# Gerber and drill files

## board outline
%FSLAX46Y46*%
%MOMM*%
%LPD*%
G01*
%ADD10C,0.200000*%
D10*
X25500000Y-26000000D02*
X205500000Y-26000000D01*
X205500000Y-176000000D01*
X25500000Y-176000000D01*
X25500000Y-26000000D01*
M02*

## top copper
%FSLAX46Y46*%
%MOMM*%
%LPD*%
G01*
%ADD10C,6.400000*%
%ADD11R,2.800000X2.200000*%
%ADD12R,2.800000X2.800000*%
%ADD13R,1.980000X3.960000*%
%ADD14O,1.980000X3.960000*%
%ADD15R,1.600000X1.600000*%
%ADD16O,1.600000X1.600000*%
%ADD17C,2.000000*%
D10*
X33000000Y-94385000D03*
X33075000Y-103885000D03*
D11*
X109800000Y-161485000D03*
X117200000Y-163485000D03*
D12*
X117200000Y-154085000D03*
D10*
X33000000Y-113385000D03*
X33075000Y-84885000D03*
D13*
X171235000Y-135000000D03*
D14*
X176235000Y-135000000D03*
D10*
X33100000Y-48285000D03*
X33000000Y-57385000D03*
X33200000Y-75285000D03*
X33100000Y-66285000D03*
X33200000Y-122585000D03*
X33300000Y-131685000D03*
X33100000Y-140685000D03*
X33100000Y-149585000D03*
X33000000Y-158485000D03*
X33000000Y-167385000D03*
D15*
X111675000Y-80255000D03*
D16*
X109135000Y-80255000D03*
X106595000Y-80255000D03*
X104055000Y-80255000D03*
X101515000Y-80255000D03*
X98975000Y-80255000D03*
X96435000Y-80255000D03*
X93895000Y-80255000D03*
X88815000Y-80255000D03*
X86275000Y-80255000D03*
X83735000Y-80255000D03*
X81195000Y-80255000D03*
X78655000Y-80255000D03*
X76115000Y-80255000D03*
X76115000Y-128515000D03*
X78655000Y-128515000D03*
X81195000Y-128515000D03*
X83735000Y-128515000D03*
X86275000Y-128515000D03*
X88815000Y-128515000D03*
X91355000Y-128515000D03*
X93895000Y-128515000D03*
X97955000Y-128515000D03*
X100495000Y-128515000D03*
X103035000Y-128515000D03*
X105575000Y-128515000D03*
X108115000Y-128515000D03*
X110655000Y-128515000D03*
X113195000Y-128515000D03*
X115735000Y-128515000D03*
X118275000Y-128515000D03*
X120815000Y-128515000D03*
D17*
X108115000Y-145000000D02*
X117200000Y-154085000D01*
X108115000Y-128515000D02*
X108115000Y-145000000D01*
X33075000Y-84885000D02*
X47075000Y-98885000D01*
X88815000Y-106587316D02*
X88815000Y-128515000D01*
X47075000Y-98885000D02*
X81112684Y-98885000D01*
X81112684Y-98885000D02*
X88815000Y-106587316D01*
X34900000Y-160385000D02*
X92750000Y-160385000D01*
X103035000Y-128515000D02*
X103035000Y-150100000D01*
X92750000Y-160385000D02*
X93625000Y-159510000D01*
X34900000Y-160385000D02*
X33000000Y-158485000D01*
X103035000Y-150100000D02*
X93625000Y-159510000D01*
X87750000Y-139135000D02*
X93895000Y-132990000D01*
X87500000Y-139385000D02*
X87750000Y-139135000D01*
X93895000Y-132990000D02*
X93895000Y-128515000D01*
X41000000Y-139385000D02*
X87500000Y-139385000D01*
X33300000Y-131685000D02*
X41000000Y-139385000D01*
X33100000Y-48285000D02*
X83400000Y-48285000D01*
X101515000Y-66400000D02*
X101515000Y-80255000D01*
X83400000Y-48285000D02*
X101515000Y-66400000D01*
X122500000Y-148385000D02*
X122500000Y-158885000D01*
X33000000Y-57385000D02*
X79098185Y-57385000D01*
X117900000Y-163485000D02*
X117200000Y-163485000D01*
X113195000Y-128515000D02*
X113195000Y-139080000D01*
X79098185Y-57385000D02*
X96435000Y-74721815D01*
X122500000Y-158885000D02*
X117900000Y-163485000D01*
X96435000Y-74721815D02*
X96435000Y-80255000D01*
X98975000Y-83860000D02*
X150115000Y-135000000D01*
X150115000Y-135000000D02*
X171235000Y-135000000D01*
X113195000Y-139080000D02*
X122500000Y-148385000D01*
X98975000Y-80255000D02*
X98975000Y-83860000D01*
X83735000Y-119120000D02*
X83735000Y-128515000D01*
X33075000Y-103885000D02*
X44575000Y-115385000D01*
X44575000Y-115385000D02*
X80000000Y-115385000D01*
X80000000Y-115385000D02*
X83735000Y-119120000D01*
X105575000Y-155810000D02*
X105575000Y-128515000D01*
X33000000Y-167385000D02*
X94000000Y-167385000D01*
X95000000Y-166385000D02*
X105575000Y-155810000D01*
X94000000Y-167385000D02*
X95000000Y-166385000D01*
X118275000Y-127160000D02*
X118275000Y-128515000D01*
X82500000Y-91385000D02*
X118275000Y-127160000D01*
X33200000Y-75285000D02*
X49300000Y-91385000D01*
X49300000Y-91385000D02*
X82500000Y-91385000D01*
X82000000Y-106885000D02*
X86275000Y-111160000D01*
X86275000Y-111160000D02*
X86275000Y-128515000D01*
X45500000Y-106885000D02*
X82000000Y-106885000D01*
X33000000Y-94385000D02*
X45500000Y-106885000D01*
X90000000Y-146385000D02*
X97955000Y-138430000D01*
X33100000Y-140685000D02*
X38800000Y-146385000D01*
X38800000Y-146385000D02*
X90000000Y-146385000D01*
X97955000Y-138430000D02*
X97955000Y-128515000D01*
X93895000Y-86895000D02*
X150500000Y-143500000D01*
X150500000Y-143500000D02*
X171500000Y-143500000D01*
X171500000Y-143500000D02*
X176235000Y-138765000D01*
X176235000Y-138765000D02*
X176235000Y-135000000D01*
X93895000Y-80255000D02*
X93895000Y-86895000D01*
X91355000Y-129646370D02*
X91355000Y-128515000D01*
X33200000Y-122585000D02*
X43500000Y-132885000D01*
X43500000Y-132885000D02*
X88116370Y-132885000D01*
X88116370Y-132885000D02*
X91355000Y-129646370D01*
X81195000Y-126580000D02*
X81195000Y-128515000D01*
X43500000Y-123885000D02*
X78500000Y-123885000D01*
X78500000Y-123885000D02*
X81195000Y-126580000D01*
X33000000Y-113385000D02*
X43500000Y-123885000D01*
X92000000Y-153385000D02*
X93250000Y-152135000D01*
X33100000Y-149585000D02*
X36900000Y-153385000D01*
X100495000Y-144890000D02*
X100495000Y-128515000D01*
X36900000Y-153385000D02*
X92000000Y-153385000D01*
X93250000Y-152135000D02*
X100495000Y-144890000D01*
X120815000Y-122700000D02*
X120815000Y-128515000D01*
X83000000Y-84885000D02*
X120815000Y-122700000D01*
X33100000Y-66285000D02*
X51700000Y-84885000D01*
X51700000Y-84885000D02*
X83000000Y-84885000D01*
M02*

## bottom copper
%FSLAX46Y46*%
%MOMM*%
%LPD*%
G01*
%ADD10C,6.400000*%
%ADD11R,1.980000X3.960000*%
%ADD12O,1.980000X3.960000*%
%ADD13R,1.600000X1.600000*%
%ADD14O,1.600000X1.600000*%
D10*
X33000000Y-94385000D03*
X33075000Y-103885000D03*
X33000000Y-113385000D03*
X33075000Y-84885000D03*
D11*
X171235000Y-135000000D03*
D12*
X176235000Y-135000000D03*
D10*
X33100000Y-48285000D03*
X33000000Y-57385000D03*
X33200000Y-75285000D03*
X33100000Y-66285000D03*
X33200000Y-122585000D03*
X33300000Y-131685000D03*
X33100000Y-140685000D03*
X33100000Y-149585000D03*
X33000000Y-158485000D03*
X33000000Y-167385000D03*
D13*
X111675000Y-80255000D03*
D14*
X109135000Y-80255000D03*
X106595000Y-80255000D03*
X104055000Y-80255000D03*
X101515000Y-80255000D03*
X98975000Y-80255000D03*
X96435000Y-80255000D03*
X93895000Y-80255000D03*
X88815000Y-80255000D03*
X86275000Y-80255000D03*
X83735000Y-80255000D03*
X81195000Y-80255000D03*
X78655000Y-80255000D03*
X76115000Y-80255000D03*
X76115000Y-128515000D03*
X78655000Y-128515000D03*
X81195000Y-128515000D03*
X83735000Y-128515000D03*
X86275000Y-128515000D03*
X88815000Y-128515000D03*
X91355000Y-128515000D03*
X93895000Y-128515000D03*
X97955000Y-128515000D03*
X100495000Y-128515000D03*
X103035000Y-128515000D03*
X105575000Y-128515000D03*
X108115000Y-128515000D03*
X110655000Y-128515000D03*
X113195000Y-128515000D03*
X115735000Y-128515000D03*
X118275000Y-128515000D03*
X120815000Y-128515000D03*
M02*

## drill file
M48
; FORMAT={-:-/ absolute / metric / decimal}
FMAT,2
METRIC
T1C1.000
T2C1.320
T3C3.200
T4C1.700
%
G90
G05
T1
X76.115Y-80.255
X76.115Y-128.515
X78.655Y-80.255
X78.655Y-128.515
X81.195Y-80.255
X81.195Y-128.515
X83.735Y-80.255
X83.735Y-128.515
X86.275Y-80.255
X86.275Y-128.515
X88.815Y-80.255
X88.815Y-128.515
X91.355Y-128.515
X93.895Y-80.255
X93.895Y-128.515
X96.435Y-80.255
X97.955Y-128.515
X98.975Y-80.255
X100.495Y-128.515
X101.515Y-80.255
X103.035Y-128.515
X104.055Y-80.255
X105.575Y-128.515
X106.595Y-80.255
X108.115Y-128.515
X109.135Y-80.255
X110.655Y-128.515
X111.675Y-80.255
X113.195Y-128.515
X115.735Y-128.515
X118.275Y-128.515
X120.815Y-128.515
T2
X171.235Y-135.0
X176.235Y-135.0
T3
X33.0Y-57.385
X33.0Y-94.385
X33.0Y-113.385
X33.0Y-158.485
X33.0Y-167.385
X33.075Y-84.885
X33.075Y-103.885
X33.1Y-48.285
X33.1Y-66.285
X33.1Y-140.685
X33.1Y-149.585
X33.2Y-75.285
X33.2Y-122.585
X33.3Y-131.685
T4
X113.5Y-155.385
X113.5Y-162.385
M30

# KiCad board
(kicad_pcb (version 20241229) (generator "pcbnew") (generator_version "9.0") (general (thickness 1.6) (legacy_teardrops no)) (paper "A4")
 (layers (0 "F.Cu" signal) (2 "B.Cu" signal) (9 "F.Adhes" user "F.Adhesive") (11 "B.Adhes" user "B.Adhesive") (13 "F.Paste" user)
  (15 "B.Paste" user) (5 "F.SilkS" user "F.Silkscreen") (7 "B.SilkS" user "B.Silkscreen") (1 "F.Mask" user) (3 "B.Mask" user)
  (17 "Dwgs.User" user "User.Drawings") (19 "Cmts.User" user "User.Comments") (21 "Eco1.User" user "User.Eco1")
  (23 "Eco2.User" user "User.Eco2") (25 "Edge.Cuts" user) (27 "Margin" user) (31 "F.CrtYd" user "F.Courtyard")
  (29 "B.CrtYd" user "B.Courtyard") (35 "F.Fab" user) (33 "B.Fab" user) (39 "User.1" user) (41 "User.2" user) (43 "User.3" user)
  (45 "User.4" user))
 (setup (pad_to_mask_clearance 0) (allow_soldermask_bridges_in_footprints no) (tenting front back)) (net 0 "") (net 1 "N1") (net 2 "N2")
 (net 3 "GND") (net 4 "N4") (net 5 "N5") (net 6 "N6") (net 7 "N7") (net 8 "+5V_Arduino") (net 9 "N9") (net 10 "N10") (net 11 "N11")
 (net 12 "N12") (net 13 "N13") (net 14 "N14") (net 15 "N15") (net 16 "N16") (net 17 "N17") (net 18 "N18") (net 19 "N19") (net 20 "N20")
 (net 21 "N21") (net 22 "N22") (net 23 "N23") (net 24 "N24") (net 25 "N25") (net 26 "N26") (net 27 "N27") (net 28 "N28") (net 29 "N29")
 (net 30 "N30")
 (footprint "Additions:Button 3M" (layer "F.Cu") (at 36.8 94.485)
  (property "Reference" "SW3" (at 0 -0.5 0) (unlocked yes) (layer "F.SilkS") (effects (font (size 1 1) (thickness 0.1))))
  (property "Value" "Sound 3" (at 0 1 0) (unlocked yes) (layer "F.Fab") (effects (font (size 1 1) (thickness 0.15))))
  (pad "2" thru_hole circle (at -3.8 -0.1) (size 6.4 6.4) (drill 3.2) (layers "*.Cu" "*.Mask") (remove_unused_layers no) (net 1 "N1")
   (zone_connect 2)))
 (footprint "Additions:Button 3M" (layer "F.Cu") (at 36.875 103.985)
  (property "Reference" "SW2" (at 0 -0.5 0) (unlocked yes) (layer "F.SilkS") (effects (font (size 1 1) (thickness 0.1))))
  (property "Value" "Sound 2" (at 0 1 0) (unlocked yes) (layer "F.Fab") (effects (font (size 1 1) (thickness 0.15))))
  (pad "2" thru_hole circle (at -3.8 -0.1) (size 6.4 6.4) (drill 3.2) (layers "*.Cu" "*.Mask") (remove_unused_layers no) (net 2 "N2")
   (zone_connect 2)))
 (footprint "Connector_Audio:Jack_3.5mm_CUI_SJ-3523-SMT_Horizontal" (layer "F.Cu") (at 113.5 159.885 180)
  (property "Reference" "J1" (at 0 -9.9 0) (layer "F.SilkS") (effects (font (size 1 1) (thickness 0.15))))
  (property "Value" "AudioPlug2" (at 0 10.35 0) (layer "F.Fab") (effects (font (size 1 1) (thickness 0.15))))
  (pad "" np_thru_hole circle (at 0 -2.5 180) (size 1.7 1.7) (drill 1.7) (layers "*.Cu" "*.Mask"))
  (pad "" np_thru_hole circle (at 0 4.5 180) (size 1.7 1.7) (drill 1.7) (layers "*.Cu" "*.Mask"))
  (pad "R" smd rect (at 3.7 -1.6 180) (size 2.8 2.2) (layers "F.Cu" "F.Mask" "F.Paste"))
  (pad "S" smd rect (at -3.7 -3.6 180) (size 2.8 2.2) (layers "F.Cu" "F.Mask" "F.Paste") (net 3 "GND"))
  (pad "T" smd rect (at -3.7 5.8 180) (size 2.8 2.8) (layers "F.Cu" "F.Mask" "F.Paste") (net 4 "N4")))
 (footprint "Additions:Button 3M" (layer "F.Cu") (at 36.8 113.485)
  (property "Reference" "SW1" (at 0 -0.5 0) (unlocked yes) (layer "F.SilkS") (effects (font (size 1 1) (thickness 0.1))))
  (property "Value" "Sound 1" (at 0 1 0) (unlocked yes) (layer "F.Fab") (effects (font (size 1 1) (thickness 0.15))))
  (pad "2" thru_hole circle (at -3.8 -0.1) (size 6.4 6.4) (drill 3.2) (layers "*.Cu" "*.Mask") (remove_unused_layers no) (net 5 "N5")
   (zone_connect 2)))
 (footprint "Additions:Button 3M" (layer "F.Cu") (at 36.875 84.985)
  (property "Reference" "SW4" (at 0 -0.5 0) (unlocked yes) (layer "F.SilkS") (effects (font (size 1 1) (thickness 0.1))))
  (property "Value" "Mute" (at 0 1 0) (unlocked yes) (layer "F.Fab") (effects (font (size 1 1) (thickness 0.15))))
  (pad "2" thru_hole circle (at -3.8 -0.1) (size 6.4 6.4) (drill 3.2) (layers "*.Cu" "*.Mask") (remove_unused_layers no) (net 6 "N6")
   (zone_connect 2)))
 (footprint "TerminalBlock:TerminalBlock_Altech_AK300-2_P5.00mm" (layer "F.Cu") (at 171.235 135)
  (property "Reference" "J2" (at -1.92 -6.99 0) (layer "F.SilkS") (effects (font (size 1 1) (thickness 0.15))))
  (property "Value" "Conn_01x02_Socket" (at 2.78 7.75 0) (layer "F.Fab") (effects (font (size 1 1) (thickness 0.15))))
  (pad "1" thru_hole rect (at 0 0) (size 1.98 3.96) (drill 1.32) (layers "*.Cu" "*.Mask") (remove_unused_layers no) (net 3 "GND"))
  (pad "2" thru_hole oval (at 5 0) (size 1.98 3.96) (drill 1.32) (layers "*.Cu" "*.Mask") (remove_unused_layers no) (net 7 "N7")))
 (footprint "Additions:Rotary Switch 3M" (layer "F.Cu") (at 33 63.785 90)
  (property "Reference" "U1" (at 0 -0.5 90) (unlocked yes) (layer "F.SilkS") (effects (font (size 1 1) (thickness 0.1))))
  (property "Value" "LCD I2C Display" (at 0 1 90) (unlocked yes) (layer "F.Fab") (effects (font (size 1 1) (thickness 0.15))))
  (pad "1" thru_hole circle (at 15.5 0.1 90) (size 6.4 6.4) (drill 3.2) (layers "*.Cu" "*.Mask") (remove_unused_layers no)
   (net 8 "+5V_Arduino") (zone_connect 2))
  (pad "2" thru_hole circle (at 6.4 0 90) (size 6.4 6.4) (drill 3.2) (layers "*.Cu" "*.Mask") (remove_unused_layers no) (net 3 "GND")
   (zone_connect 2))
  (pad "3" thru_hole circle (at -11.5 0.2 90) (size 6.4 6.4) (drill 3.2) (layers "*.Cu" "*.Mask") (remove_unused_layers no) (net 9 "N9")
   (zone_connect 2))
  (pad "4" thru_hole circle (at -2.5 0.1 90) (size 6.4 6.4) (drill 3.2) (layers "*.Cu" "*.Mask") (remove_unused_layers no) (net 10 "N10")
   (zone_connect 2)))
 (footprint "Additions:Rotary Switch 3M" (layer "F.Cu") (at 33.1 153.885 90)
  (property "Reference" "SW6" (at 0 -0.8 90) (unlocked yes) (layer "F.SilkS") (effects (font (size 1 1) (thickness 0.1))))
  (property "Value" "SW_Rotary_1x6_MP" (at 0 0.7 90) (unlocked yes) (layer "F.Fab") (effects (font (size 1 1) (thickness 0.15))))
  (pad "1" thru_hole circle (at 31.3 0.1 90) (size 6.4 6.4) (drill 3.2) (layers "*.Cu" "*.Mask") (remove_unused_layers no) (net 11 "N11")
   (zone_connect 2))
  (pad "2" thru_hole circle (at 22.2 0.2 90) (size 6.4 6.4) (drill 3.2) (layers "*.Cu" "*.Mask") (remove_unused_layers no) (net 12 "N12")
   (zone_connect 2))
  (pad "3" thru_hole circle (at 13.2 0 90) (size 6.4 6.4) (drill 3.2) (layers "*.Cu" "*.Mask") (remove_unused_layers no) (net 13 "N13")
   (zone_connect 2))
  (pad "4" thru_hole circle (at 4.3 0 90) (size 6.4 6.4) (drill 3.2) (layers "*.Cu" "*.Mask") (remove_unused_layers no) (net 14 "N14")
   (zone_connect 2))
  (pad "5" thru_hole circle (at -4.6 -0.1 90) (size 6.4 6.4) (drill 3.2) (layers "*.Cu" "*.Mask") (remove_unused_layers no) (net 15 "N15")
   (zone_connect 2))
  (pad "6" thru_hole circle (at -13.5 -0.1 90) (size 6.4 6.4) (drill 3.2) (layers "*.Cu" "*.Mask") (remove_unused_layers no) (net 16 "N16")
   (zone_connect 2)))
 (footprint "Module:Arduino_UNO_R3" (layer "B.Cu") (at 111.675 80.255 180)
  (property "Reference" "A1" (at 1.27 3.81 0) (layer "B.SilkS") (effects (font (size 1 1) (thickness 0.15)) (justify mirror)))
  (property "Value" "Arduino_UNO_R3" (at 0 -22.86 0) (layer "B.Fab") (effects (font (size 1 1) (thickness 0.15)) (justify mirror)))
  (pad "1" thru_hole rect (at 0 0 90) (size 1.6 1.6) (drill 1) (layers "*.Cu" "*.Mask") (remove_unused_layers no) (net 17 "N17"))
  (pad "2" thru_hole oval (at 2.54 0 90) (size 1.6 1.6) (drill 1) (layers "*.Cu" "*.Mask") (remove_unused_layers no) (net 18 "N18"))
  (pad "3" thru_hole oval (at 5.08 0 90) (size 1.6 1.6) (drill 1) (layers "*.Cu" "*.Mask") (remove_unused_layers no) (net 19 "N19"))
  (pad "4" thru_hole oval (at 7.62 0 90) (size 1.6 1.6) (drill 1) (layers "*.Cu" "*.Mask") (remove_unused_layers no) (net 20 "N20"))
  (pad "5" thru_hole oval (at 10.16 0 90) (size 1.6 1.6) (drill 1) (layers "*.Cu" "*.Mask") (remove_unused_layers no) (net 8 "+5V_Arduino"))
  (pad "6" thru_hole oval (at 12.7 0 90) (size 1.6 1.6) (drill 1) (layers "*.Cu" "*.Mask") (remove_unused_layers no) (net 3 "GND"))
  (pad "7" thru_hole oval (at 15.24 0 90) (size 1.6 1.6) (drill 1) (layers "*.Cu" "*.Mask") (remove_unused_layers no) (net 3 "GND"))
  (pad "8" thru_hole oval (at 17.78 0 90) (size 1.6 1.6) (drill 1) (layers "*.Cu" "*.Mask") (remove_unused_layers no) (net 7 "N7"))
  (pad "9" thru_hole oval (at 22.86 0 90) (size 1.6 1.6) (drill 1) (layers "*.Cu" "*.Mask") (remove_unused_layers no) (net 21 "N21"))
  (pad "10" thru_hole oval (at 25.4 0 90) (size 1.6 1.6) (drill 1) (layers "*.Cu" "*.Mask") (remove_unused_layers no) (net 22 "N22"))
  (pad "11" thru_hole oval (at 27.94 0 90) (size 1.6 1.6) (drill 1) (layers "*.Cu" "*.Mask") (remove_unused_layers no) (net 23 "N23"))
  (pad "12" thru_hole oval (at 30.48 0 90) (size 1.6 1.6) (drill 1) (layers "*.Cu" "*.Mask") (remove_unused_layers no) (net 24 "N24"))
  (pad "13" thru_hole oval (at 33.02 0 90) (size 1.6 1.6) (drill 1) (layers "*.Cu" "*.Mask") (remove_unused_layers no) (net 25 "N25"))
  (pad "14" thru_hole oval (at 35.56 0 90) (size 1.6 1.6) (drill 1) (layers "*.Cu" "*.Mask") (remove_unused_layers no) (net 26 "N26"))
  (pad "15" thru_hole oval (at 35.56 -48.26 90) (size 1.6 1.6) (drill 1) (layers "*.Cu" "*.Mask") (remove_unused_layers no) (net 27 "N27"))
  (pad "16" thru_hole oval (at 33.02 -48.26 90) (size 1.6 1.6) (drill 1) (layers "*.Cu" "*.Mask") (remove_unused_layers no) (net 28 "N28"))
  (pad "17" thru_hole oval (at 30.48 -48.26 90) (size 1.6 1.6) (drill 1) (layers "*.Cu" "*.Mask") (remove_unused_layers no) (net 5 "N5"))
  (pad "18" thru_hole oval (at 27.94 -48.26 90) (size 1.6 1.6) (drill 1) (layers "*.Cu" "*.Mask") (remove_unused_layers no) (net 2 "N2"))
  (pad "19" thru_hole oval (at 25.4 -48.26 90) (size 1.6 1.6) (drill 1) (layers "*.Cu" "*.Mask") (remove_unused_layers no) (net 1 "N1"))
  (pad "20" thru_hole oval (at 22.86 -48.26 90) (size 1.6 1.6) (drill 1) (layers "*.Cu" "*.Mask") (remove_unused_layers no) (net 6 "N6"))
  (pad "21" thru_hole oval (at 20.32 -48.26 90) (size 1.6 1.6) (drill 1) (layers "*.Cu" "*.Mask") (remove_unused_layers no) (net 11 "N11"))
  (pad "22" thru_hole oval (at 17.78 -48.26 90) (size 1.6 1.6) (drill 1) (layers "*.Cu" "*.Mask") (remove_unused_layers no) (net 12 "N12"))
  (pad "23" thru_hole oval (at 13.72 -48.26 90) (size 1.6 1.6) (drill 1) (layers "*.Cu" "*.Mask") (remove_unused_layers no) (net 13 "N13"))
  (pad "24" thru_hole oval (at 11.18 -48.26 90) (size 1.6 1.6) (drill 1) (layers "*.Cu" "*.Mask") (remove_unused_layers no) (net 14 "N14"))
  (pad "25" thru_hole oval (at 8.64 -48.26 90) (size 1.6 1.6) (drill 1) (layers "*.Cu" "*.Mask") (remove_unused_layers no) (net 15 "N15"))
  (pad "26" thru_hole oval (at 6.1 -48.26 90) (size 1.6 1.6) (drill 1) (layers "*.Cu" "*.Mask") (remove_unused_layers no) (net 16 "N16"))
  (pad "27" thru_hole oval (at 3.56 -48.26 90) (size 1.6 1.6) (drill 1) (layers "*.Cu" "*.Mask") (remove_unused_layers no) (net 4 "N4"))
  (pad "28" thru_hole oval (at 1.02 -48.26 90) (size 1.6 1.6) (drill 1) (layers "*.Cu" "*.Mask") (remove_unused_layers no) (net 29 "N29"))
  (pad "29" thru_hole oval (at -1.52 -48.26 90) (size 1.6 1.6) (drill 1) (layers "*.Cu" "*.Mask") (remove_unused_layers no) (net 3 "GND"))
  (pad "30" thru_hole oval (at -4.06 -48.26 90) (size 1.6 1.6) (drill 1) (layers "*.Cu" "*.Mask") (remove_unused_layers no) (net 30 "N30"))
  (pad "31" thru_hole oval (at -6.6 -48.26 90) (size 1.6 1.6) (drill 1) (layers "*.Cu" "*.Mask") (remove_unused_layers no) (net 9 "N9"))
  (pad "32" thru_hole oval (at -9.14 -48.26 90) (size 1.6 1.6) (drill 1) (layers "*.Cu" "*.Mask") (remove_unused_layers no) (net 10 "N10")))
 (gr_rect (start 25.5 26) (end 205.5 176) (stroke (width 0.2) (type solid)) (fill no) (layer "Edge.Cuts"))
 (segment (start 108.115 145) (end 117.2 154.085) (width 2) (layer "F.Cu") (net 4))
 (segment (start 108.115 128.515) (end 108.115 145) (width 2) (layer "F.Cu") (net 4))
 (segment (start 33.075 84.885) (end 47.075 98.885) (width 2) (layer "F.Cu") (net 6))
 (segment (start 88.815 106.587316) (end 88.815 128.515) (width 2) (layer "F.Cu") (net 6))
 (segment (start 47.075 98.885) (end 81.112684 98.885) (width 2) (layer "F.Cu") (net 6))
 (segment (start 81.112684 98.885) (end 88.815 106.587316) (width 2) (layer "F.Cu") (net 6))
 (segment (start 34.9 160.385) (end 92.75 160.385) (width 2) (layer "F.Cu") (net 15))
 (segment (start 103.035 128.515) (end 103.035 150.1) (width 2) (layer "F.Cu") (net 15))
 (segment (start 92.75 160.385) (end 93.625 159.51) (width 2) (layer "F.Cu") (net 15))
 (segment (start 34.9 160.385) (end 33 158.485) (width 2) (layer "F.Cu") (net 15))
 (segment (start 103.035 150.1) (end 93.625 159.51) (width 2) (layer "F.Cu") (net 15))
 (segment (start 87.75 139.135) (end 93.895 132.99) (width 2) (layer "F.Cu") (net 12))
 (segment (start 87.5 139.385) (end 87.75 139.135) (width 2) (layer "F.Cu") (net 12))
 (segment (start 93.895 132.99) (end 93.895 128.515) (width 2) (layer "F.Cu") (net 12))
 (segment (start 41 139.385) (end 87.5 139.385) (width 2) (layer "F.Cu") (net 12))
 (segment (start 33.3 131.685) (end 41 139.385) (width 2) (layer "F.Cu") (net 12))
 (segment (start 33.1 48.285) (end 83.4 48.285) (width 2) (layer "F.Cu") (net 8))
 (segment (start 101.515 66.4) (end 101.515 80.255) (width 2) (layer "F.Cu") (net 8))
 (segment (start 83.4 48.285) (end 101.515 66.4) (width 2) (layer "F.Cu") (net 8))
 (segment (start 122.5 148.385) (end 122.5 158.885) (width 2) (layer "F.Cu") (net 3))
 (segment (start 33 57.385) (end 79.098185 57.385) (width 2) (layer "F.Cu") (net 3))
 (segment (start 117.9 163.485) (end 117.2 163.485) (width 2) (layer "F.Cu") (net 3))
 (segment (start 113.195 128.515) (end 113.195 139.08) (width 2) (layer "F.Cu") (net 3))
 (segment (start 79.098185 57.385) (end 96.435 74.721815) (width 2) (layer "F.Cu") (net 3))
 (segment (start 122.5 158.885) (end 117.9 163.485) (width 2) (layer "F.Cu") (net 3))
 (segment (start 96.435 74.721815) (end 96.435 80.255) (width 2) (layer "F.Cu") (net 3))
 (segment (start 98.975 83.86) (end 150.115 135) (width 2) (layer "F.Cu") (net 3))
 (segment (start 150.115 135) (end 171.235 135) (width 2) (layer "F.Cu") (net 3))
 (segment (start 113.195 139.08) (end 122.5 148.385) (width 2) (layer "F.Cu") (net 3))
 (segment (start 98.975 80.255) (end 98.975 83.86) (width 2) (layer "F.Cu") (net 3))
 (segment (start 83.735 119.12) (end 83.735 128.515) (width 2) (layer "F.Cu") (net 2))
 (segment (start 33.075 103.885) (end 44.575 115.385) (width 2) (layer "F.Cu") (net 2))
 (segment (start 44.575 115.385) (end 80 115.385) (width 2) (layer "F.Cu") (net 2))
 (segment (start 80 115.385) (end 83.735 119.12) (width 2) (layer "F.Cu") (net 2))
 (segment (start 105.575 155.81) (end 105.575 128.515) (width 2) (layer "F.Cu") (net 16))
 (segment (start 33 167.385) (end 94 167.385) (width 2) (layer "F.Cu") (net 16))
 (segment (start 95 166.385) (end 105.575 155.81) (width 2) (layer "F.Cu") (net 16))
 (segment (start 94 167.385) (end 95 166.385) (width 2) (layer "F.Cu") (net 16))
 (segment (start 118.275 127.16) (end 118.275 128.515) (width 2) (layer "F.Cu") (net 9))
 (segment (start 82.5 91.385) (end 118.275 127.16) (width 2) (layer "F.Cu") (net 9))
 (segment (start 33.2 75.285) (end 49.3 91.385) (width 2) (layer "F.Cu") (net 9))
 (segment (start 49.3 91.385) (end 82.5 91.385) (width 2) (layer "F.Cu") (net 9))
 (segment (start 82 106.885) (end 86.275 111.16) (width 2) (layer "F.Cu") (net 1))
 (segment (start 86.275 111.16) (end 86.275 128.515) (width 2) (layer "F.Cu") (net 1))
 (segment (start 45.5 106.885) (end 82 106.885) (width 2) (layer "F.Cu") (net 1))
 (segment (start 33 94.385) (end 45.5 106.885) (width 2) (layer "F.Cu") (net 1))
 (segment (start 90 146.385) (end 97.955 138.43) (width 2) (layer "F.Cu") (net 13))
 (segment (start 33.1 140.685) (end 38.8 146.385) (width 2) (layer "F.Cu") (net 13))
 (segment (start 38.8 146.385) (end 90 146.385) (width 2) (layer "F.Cu") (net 13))
 (segment (start 97.955 138.43) (end 97.955 128.515) (width 2) (layer "F.Cu") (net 13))
 (segment (start 93.895 86.895) (end 150.5 143.5) (width 2) (layer "F.Cu") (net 7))
 (segment (start 150.5 143.5) (end 171.5 143.5) (width 2) (layer "F.Cu") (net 7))
 (segment (start 171.5 143.5) (end 176.235 138.765) (width 2) (layer "F.Cu") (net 7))
 (segment (start 176.235 138.765) (end 176.235 135) (width 2) (layer "F.Cu") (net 7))
 (segment (start 93.895 80.255) (end 93.895 86.895) (width 2) (layer "F.Cu") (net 7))
 (segment (start 91.355 129.64637) (end 91.355 128.515) (width 2) (layer "F.Cu") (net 11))
 (segment (start 33.2 122.585) (end 43.5 132.885) (width 2) (layer "F.Cu") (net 11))
 (segment (start 43.5 132.885) (end 88.11637 132.885) (width 2) (layer "F.Cu") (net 11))
 (segment (start 88.11637 132.885) (end 91.355 129.64637) (width 2) (layer "F.Cu") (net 11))
 (segment (start 81.195 126.58) (end 81.195 128.515) (width 2) (layer "F.Cu") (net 5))
 (segment (start 43.5 123.885) (end 78.5 123.885) (width 2) (layer "F.Cu") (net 5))
 (segment (start 78.5 123.885) (end 81.195 126.58) (width 2) (layer "F.Cu") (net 5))
 (segment (start 33 113.385) (end 43.5 123.885) (width 2) (layer "F.Cu") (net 5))
 (segment (start 92 153.385) (end 93.25 152.135) (width 2) (layer "F.Cu") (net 14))
 (segment (start 33.1 149.585) (end 36.9 153.385) (width 2) (layer "F.Cu") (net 14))
 (segment (start 100.495 144.89) (end 100.495 128.515) (width 2) (layer "F.Cu") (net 14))
 (segment (start 36.9 153.385) (end 92 153.385) (width 2) (layer "F.Cu") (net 14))
 (segment (start 93.25 152.135) (end 100.495 144.89) (width 2) (layer "F.Cu") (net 14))
 (segment (start 120.815 122.7) (end 120.815 128.515) (width 2) (layer "F.Cu") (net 10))
 (segment (start 83 84.885) (end 120.815 122.7) (width 2) (layer "F.Cu") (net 10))
 (segment (start 33.1 66.285) (end 51.7 84.885) (width 2) (layer "F.Cu") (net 10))
 (segment (start 51.7 84.885) (end 83 84.885) (width 2) (layer "F.Cu") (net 10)))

